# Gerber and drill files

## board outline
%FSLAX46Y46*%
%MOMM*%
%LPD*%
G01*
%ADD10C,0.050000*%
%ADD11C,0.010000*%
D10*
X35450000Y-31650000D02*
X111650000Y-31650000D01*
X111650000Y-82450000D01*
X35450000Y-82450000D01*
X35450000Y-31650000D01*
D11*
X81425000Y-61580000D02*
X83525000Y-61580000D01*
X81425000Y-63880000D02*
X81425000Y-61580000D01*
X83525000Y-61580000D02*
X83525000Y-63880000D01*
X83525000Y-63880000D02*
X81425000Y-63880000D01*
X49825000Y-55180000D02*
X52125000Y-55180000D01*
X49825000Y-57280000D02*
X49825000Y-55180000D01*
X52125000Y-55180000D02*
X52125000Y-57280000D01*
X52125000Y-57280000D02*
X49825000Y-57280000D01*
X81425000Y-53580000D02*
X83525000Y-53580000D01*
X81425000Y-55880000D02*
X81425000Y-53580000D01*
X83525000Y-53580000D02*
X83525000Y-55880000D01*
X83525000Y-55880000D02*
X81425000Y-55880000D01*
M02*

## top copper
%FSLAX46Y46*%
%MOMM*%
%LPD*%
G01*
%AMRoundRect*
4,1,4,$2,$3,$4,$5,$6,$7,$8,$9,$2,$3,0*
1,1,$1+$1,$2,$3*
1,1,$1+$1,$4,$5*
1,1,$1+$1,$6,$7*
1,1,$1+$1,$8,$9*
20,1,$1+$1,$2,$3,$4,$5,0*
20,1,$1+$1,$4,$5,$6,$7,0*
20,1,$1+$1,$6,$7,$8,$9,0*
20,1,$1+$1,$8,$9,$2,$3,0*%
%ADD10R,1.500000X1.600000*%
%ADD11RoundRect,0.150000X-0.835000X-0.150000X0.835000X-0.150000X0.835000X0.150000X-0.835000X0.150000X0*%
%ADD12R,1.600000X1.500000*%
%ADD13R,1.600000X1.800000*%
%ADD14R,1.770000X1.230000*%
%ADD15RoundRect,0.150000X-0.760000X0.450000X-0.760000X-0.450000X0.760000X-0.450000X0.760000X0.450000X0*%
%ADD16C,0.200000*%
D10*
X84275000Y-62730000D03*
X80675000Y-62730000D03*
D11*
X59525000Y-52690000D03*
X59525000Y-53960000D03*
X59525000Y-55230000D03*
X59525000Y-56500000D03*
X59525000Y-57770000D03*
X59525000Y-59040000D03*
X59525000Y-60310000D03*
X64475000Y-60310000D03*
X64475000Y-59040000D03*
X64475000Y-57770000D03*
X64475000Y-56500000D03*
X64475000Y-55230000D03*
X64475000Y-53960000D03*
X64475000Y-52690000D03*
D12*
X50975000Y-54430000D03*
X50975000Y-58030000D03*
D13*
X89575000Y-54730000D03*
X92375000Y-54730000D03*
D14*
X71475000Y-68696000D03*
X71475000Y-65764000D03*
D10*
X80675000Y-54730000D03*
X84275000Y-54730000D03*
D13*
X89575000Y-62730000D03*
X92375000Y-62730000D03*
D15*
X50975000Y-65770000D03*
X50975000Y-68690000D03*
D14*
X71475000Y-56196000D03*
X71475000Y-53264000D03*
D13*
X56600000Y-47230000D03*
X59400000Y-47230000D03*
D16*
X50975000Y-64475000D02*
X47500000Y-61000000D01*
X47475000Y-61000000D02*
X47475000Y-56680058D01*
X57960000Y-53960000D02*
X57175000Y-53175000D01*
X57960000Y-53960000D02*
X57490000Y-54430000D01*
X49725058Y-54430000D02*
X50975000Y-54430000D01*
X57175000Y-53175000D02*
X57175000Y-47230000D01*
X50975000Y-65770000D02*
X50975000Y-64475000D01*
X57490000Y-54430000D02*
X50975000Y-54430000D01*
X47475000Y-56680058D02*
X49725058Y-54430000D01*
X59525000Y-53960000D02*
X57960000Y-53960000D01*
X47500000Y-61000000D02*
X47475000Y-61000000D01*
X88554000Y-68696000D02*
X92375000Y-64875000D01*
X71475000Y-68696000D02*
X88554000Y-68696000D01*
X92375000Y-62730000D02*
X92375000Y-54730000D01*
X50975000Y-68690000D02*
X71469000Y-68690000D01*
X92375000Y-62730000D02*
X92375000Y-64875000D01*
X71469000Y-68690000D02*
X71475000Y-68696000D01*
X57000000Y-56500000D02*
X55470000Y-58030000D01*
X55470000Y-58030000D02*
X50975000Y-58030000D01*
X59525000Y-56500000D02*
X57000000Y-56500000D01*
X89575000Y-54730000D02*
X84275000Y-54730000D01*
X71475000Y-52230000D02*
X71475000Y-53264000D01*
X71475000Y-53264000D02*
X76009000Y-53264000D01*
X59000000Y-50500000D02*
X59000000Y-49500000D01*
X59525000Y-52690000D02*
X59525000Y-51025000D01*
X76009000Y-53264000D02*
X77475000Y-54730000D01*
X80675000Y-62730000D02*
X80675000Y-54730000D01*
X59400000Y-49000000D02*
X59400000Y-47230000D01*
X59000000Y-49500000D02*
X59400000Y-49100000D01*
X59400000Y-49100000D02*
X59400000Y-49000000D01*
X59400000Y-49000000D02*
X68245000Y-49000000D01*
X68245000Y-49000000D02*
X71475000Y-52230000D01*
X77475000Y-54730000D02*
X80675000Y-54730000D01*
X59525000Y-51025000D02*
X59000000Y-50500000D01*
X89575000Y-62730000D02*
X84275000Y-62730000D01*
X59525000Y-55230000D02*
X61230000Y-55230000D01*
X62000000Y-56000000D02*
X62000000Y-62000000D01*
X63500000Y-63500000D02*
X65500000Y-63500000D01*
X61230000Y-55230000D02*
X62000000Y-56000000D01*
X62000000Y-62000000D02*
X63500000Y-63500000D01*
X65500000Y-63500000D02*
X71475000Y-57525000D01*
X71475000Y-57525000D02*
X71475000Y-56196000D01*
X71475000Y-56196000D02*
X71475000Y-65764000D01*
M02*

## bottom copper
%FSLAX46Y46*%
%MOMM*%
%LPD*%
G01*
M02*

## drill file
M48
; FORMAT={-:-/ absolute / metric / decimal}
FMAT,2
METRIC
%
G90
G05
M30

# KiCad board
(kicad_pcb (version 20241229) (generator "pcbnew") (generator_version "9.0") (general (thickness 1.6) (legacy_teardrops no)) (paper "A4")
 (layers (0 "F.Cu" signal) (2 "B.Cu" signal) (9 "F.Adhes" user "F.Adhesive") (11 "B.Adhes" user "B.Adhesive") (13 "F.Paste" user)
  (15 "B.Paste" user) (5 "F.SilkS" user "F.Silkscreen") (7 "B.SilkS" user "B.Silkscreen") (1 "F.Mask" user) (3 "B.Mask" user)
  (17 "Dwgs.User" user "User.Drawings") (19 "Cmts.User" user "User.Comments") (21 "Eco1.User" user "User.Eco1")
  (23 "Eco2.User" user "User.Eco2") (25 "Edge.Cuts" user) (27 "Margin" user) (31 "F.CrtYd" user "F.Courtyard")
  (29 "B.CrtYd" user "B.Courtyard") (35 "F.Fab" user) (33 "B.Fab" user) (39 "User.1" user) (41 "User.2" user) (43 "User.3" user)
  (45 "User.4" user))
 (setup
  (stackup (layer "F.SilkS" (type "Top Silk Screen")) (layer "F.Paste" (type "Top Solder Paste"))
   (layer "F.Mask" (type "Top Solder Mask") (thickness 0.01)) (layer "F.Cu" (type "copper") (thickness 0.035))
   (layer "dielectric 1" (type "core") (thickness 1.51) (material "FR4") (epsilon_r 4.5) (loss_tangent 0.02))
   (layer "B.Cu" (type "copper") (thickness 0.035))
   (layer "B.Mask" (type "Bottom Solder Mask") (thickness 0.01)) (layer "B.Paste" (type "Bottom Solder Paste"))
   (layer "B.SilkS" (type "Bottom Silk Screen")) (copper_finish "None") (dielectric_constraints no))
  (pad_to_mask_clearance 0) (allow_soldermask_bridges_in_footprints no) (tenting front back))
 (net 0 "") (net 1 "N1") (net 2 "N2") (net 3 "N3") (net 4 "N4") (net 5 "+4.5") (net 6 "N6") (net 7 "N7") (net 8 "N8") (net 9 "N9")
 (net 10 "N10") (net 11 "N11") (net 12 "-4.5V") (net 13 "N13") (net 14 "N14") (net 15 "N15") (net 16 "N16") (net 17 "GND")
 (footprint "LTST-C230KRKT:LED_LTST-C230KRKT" (layer "F.Cu") (at 82.475 62.73)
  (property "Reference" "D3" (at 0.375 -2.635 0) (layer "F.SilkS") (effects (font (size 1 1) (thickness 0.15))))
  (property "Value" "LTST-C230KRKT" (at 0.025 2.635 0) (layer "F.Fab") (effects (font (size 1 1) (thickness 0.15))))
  (fp_line (start -1.05 -1.15) (end 1.05 -1.15) (stroke (width 0.01) (type solid)) (layer "Edge.Cuts"))
  (fp_line (start -1.05 1.15) (end -1.05 -1.15) (stroke (width 0.01) (type solid)) (layer "Edge.Cuts"))
  (fp_line (start 1.05 -1.15) (end 1.05 1.15) (stroke (width 0.01) (type solid)) (layer "Edge.Cuts"))
  (fp_line (start 1.05 1.15) (end -1.05 1.15) (stroke (width 0.01) (type solid)) (layer "Edge.Cuts"))
  (pad "A" smd rect (at 1.8 0) (size 1.5 1.6) (layers "F.Cu" "F.Mask" "F.Paste") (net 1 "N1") (solder_mask_margin 0.102))
  (pad "C" smd rect (at -1.8 0) (size 1.5 1.6) (layers "F.Cu" "F.Mask" "F.Paste") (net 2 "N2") (solder_mask_margin 0.102)))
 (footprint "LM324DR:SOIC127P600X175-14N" (layer "F.Cu") (at 62 56.5)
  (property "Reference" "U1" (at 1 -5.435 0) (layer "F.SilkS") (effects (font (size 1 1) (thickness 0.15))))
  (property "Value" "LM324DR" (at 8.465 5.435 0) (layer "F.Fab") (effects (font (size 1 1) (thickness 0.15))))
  (pad "1" smd roundrect (at -2.475 -3.81) (size 1.97 0.6) (layers "F.Cu" "F.Mask" "F.Paste") (roundrect_rratio 0.25) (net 2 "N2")
   (solder_mask_margin 0.102))
  (pad "2" smd roundrect (at -2.475 -2.54) (size 1.97 0.6) (layers "F.Cu" "F.Mask" "F.Paste") (roundrect_rratio 0.25) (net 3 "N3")
   (solder_mask_margin 0.102))
  (pad "3" smd roundrect (at -2.475 -1.27) (size 1.97 0.6) (layers "F.Cu" "F.Mask" "F.Paste") (roundrect_rratio 0.25) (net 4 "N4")
   (solder_mask_margin 0.102))
  (pad "4" smd roundrect (at -2.475 0) (size 1.97 0.6) (layers "F.Cu" "F.Mask" "F.Paste") (roundrect_rratio 0.25) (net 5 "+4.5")
   (solder_mask_margin 0.102))
  (pad "5" smd roundrect (at -2.475 1.27) (size 1.97 0.6) (layers "F.Cu" "F.Mask" "F.Paste") (roundrect_rratio 0.25) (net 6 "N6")
   (solder_mask_margin 0.102))
  (pad "6" smd roundrect (at -2.475 2.54) (size 1.97 0.6) (layers "F.Cu" "F.Mask" "F.Paste") (roundrect_rratio 0.25) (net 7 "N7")
   (solder_mask_margin 0.102))
  (pad "7" smd roundrect (at -2.475 3.81) (size 1.97 0.6) (layers "F.Cu" "F.Mask" "F.Paste") (roundrect_rratio 0.25) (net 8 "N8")
   (solder_mask_margin 0.102))
  (pad "8" smd roundrect (at 2.475 3.81) (size 1.97 0.6) (layers "F.Cu" "F.Mask" "F.Paste") (roundrect_rratio 0.25) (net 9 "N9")
   (solder_mask_margin 0.102))
  (pad "9" smd roundrect (at 2.475 2.54) (size 1.97 0.6) (layers "F.Cu" "F.Mask" "F.Paste") (roundrect_rratio 0.25) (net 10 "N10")
   (solder_mask_margin 0.102))
  (pad "10" smd roundrect (at 2.475 1.27) (size 1.97 0.6) (layers "F.Cu" "F.Mask" "F.Paste") (roundrect_rratio 0.25) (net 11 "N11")
   (solder_mask_margin 0.102))
  (pad "11" smd roundrect (at 2.475 0) (size 1.97 0.6) (layers "F.Cu" "F.Mask" "F.Paste") (roundrect_rratio 0.25) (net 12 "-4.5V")
   (solder_mask_margin 0.102))
  (pad "12" smd roundrect (at 2.475 -1.27) (size 1.97 0.6) (layers "F.Cu" "F.Mask" "F.Paste") (roundrect_rratio 0.25) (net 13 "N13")
   (solder_mask_margin 0.102))
  (pad "13" smd roundrect (at 2.475 -2.54) (size 1.97 0.6) (layers "F.Cu" "F.Mask" "F.Paste") (roundrect_rratio 0.25) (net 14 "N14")
   (solder_mask_margin 0.102))
  (pad "14" smd roundrect (at 2.475 -3.81) (size 1.97 0.6) (layers "F.Cu" "F.Mask" "F.Paste") (roundrect_rratio 0.25) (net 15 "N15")
   (solder_mask_margin 0.102)))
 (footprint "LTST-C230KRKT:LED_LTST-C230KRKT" (layer "F.Cu") (at 50.975 56.23 90)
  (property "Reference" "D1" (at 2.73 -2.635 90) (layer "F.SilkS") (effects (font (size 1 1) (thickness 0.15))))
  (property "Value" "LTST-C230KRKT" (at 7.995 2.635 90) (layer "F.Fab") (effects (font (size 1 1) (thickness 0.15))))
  (fp_line (start 1.05 -1.15) (end 1.05 1.15) (stroke (width 0.01) (type solid)) (layer "Edge.Cuts"))
  (fp_line (start -1.05 -1.15) (end 1.05 -1.15) (stroke (width 0.01) (type solid)) (layer "Edge.Cuts"))
  (fp_line (start 1.05 1.15) (end -1.05 1.15) (stroke (width 0.01) (type solid)) (layer "Edge.Cuts"))
  (fp_line (start -1.05 1.15) (end -1.05 -1.15) (stroke (width 0.01) (type solid)) (layer "Edge.Cuts"))
  (pad "A" smd rect (at 1.8 0 90) (size 1.5 1.6) (layers "F.Cu" "F.Mask" "F.Paste") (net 3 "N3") (solder_mask_margin 0.102))
  (pad "C" smd rect (at -1.8 0 90) (size 1.5 1.6) (layers "F.Cu" "F.Mask" "F.Paste") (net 5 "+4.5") (solder_mask_margin 0.102)))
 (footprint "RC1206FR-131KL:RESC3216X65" (layer "F.Cu") (at 90.975 54.73)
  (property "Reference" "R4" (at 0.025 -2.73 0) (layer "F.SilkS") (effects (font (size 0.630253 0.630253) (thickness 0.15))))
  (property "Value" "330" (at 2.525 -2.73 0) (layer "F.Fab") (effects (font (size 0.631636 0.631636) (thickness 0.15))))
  (pad "1" smd rect (at -1.4 0) (size 1.6 1.8) (layers "F.Cu" "F.Mask" "F.Paste") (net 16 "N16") (solder_mask_margin 0.102))
  (pad "2" smd rect (at 1.4 0) (size 1.6 1.8) (layers "F.Cu" "F.Mask" "F.Paste") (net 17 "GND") (solder_mask_margin 0.102)))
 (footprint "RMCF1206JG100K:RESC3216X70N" (layer "F.Cu") (at 71.475 67.23 90)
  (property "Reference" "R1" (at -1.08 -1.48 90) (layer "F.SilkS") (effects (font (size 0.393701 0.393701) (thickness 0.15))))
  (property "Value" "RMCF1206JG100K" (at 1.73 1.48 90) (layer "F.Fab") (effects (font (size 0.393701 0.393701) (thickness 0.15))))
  (pad "1" smd rect (at -1.466 0 90) (size 1.23 1.77) (layers "F.Cu" "F.Mask" "F.Paste") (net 17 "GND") (solder_mask_margin 0.102))
  (pad "2" smd rect (at 1.466 0 90) (size 1.23 1.77) (layers "F.Cu" "F.Mask" "F.Paste") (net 4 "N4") (solder_mask_margin 0.102)))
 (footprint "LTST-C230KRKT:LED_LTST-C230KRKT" (layer "F.Cu") (at 82.475 54.73 180)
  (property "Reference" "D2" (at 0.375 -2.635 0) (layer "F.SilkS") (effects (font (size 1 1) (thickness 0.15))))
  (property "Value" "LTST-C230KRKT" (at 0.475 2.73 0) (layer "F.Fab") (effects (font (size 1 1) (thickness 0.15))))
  (fp_line (start 1.05 1.15) (end -1.05 1.15) (stroke (width 0.01) (type solid)) (layer "Edge.Cuts"))
  (fp_line (start 1.05 -1.15) (end 1.05 1.15) (stroke (width 0.01) (type solid)) (layer "Edge.Cuts"))
  (fp_line (start -1.05 1.15) (end -1.05 -1.15) (stroke (width 0.01) (type solid)) (layer "Edge.Cuts"))
  (fp_line (start -1.05 -1.15) (end 1.05 -1.15) (stroke (width 0.01) (type solid)) (layer "Edge.Cuts"))
  (pad "A" smd rect (at 1.8 0 180) (size 1.5 1.6) (layers "F.Cu" "F.Mask" "F.Paste") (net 2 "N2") (solder_mask_margin 0.102))
  (pad "C" smd rect (at -1.8 0 180) (size 1.5 1.6) (layers "F.Cu" "F.Mask" "F.Paste") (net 16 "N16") (solder_mask_margin 0.102)))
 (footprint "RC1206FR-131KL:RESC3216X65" (layer "F.Cu") (at 90.975 62.73)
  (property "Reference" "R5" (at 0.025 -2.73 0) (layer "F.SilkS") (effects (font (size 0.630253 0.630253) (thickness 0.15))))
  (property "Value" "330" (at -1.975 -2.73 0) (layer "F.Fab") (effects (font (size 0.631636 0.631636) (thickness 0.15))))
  (pad "1" smd rect (at -1.4 0) (size 1.6 1.8) (layers "F.Cu" "F.Mask" "F.Paste") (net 1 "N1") (solder_mask_margin 0.102))
  (pad "2" smd rect (at 1.4 0) (size 1.6 1.8) (layers "F.Cu" "F.Mask" "F.Paste") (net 17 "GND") (solder_mask_margin 0.102)))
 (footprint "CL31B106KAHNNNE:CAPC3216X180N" (layer "F.Cu") (at 50.975 67.23 -90)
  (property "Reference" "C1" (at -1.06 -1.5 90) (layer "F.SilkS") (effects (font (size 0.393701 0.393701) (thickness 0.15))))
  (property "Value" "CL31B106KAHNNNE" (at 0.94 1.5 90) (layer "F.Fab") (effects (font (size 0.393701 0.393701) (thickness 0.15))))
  (pad "1" smd roundrect (at -1.46 0 270) (size 1.2 1.82) (layers "F.Cu" "F.Mask" "F.Paste") (roundrect_rratio 0.125) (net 3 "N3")
   (solder_mask_margin 0.102))
  (pad "2" smd roundrect (at 1.46 0 270) (size 1.2 1.82) (layers "F.Cu" "F.Mask" "F.Paste") (roundrect_rratio 0.125) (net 17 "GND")
   (solder_mask_margin 0.102)))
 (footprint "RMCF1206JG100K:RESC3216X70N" (layer "F.Cu") (at 71.475 54.73 90)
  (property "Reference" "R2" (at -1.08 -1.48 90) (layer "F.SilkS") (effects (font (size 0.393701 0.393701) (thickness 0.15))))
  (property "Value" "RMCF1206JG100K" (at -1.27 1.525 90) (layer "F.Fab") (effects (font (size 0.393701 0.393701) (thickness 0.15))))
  (pad "1" smd rect (at -1.466 0 90) (size 1.23 1.77) (layers "F.Cu" "F.Mask" "F.Paste") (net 4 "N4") (solder_mask_margin 0.102))
  (pad "2" smd rect (at 1.466 0 90) (size 1.23 1.77) (layers "F.Cu" "F.Mask" "F.Paste") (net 2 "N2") (solder_mask_margin 0.102)))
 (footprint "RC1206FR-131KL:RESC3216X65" (layer "F.Cu") (at 58 47.23)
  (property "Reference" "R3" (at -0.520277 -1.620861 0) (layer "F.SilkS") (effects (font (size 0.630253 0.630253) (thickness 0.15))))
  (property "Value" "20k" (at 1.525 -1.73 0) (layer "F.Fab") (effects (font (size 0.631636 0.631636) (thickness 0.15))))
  (pad "1" smd rect (at -1.4 0) (size 1.6 1.8) (layers "F.Cu" "F.Mask" "F.Paste") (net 3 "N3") (solder_mask_margin 0.102))
  (pad "2" smd rect (at 1.4 0) (size 1.6 1.8) (layers "F.Cu" "F.Mask" "F.Paste") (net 2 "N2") (solder_mask_margin 0.102)))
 (gr_rect (start 35.45 31.65) (end 111.65 82.45) (stroke (width 0.05) (type solid)) (fill no) (layer "Edge.Cuts"))
 (segment (start 50.975 64.475) (end 47.5 61) (width 0.2) (layer "F.Cu") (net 3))
 (segment (start 47.475 61) (end 47.475 56.680058) (width 0.2) (layer "F.Cu") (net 3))
 (segment (start 57.96 53.96) (end 57.175 53.175) (width 0.2) (layer "F.Cu") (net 3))
 (segment (start 57.96 53.96) (end 57.49 54.43) (width 0.2) (layer "F.Cu") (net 3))
 (segment (start 49.725058 54.43) (end 50.975 54.43) (width 0.2) (layer "F.Cu") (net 3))
 (segment (start 57.175 53.175) (end 57.175 47.23) (width 0.2) (layer "F.Cu") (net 3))
 (segment (start 50.975 65.77) (end 50.975 64.475) (width 0.2) (layer "F.Cu") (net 3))
 (segment (start 57.49 54.43) (end 50.975 54.43) (width 0.2) (layer "F.Cu") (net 3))
 (segment (start 47.475 56.680058) (end 49.725058 54.43) (width 0.2) (layer "F.Cu") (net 3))
 (segment (start 59.525 53.96) (end 57.96 53.96) (width 0.2) (layer "F.Cu") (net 3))
 (segment (start 47.5 61) (end 47.475 61) (width 0.2) (layer "F.Cu") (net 3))
 (segment (start 88.554 68.696) (end 92.375 64.875) (width 0.2) (layer "F.Cu") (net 17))
 (segment (start 71.475 68.696) (end 88.554 68.696) (width 0.2) (layer "F.Cu") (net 17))
 (segment (start 92.375 62.73) (end 92.375 54.73) (width 0.2) (layer "F.Cu") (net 17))
 (segment (start 50.975 68.69) (end 71.469 68.69) (width 0.2) (layer "F.Cu") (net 17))
 (segment (start 92.375 62.73) (end 92.375 64.875) (width 0.2) (layer "F.Cu") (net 17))
 (segment (start 71.469 68.69) (end 71.475 68.696) (width 0.2) (layer "F.Cu") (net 17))
 (segment (start 57 56.5) (end 55.47 58.03) (width 0.2) (layer "F.Cu") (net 5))
 (segment (start 55.47 58.03) (end 50.975 58.03) (width 0.2) (layer "F.Cu") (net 5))
 (segment (start 59.525 56.5) (end 57 56.5) (width 0.2) (layer "F.Cu") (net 5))
 (segment (start 89.575 54.73) (end 84.275 54.73) (width 0.2) (layer "F.Cu") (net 16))
 (segment (start 71.475 52.23) (end 71.475 53.264) (width 0.2) (layer "F.Cu") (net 2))
 (segment (start 71.475 53.264) (end 76.009 53.264) (width 0.2) (layer "F.Cu") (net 2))
 (segment (start 59 50.5) (end 59 49.5) (width 0.2) (layer "F.Cu") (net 2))
 (segment (start 59.525 52.69) (end 59.525 51.025) (width 0.2) (layer "F.Cu") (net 2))
 (segment (start 76.009 53.264) (end 77.475 54.73) (width 0.2) (layer "F.Cu") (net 2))
 (segment (start 80.675 62.73) (end 80.675 54.73) (width 0.2) (layer "F.Cu") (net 2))
 (segment (start 59.4 49) (end 59.4 47.23) (width 0.2) (layer "F.Cu") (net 2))
 (segment (start 59 49.5) (end 59.4 49.1) (width 0.2) (layer "F.Cu") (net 2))
 (segment (start 59.4 49.1) (end 59.4 49) (width 0.2) (layer "F.Cu") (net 2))
 (segment (start 59.4 49) (end 68.245 49) (width 0.2) (layer "F.Cu") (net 2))
 (segment (start 68.245 49) (end 71.475 52.23) (width 0.2) (layer "F.Cu") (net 2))
 (segment (start 77.475 54.73) (end 80.675 54.73) (width 0.2) (layer "F.Cu") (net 2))
 (segment (start 59.525 51.025) (end 59 50.5) (width 0.2) (layer "F.Cu") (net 2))
 (segment (start 89.575 62.73) (end 84.275 62.73) (width 0.2) (layer "F.Cu") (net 1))
 (segment (start 59.525 55.23) (end 61.23 55.23) (width 0.2) (layer "F.Cu") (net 4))
 (segment (start 62 56) (end 62 62) (width 0.2) (layer "F.Cu") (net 4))
 (segment (start 63.5 63.5) (end 65.5 63.5) (width 0.2) (layer "F.Cu") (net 4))
 (segment (start 61.23 55.23) (end 62 56) (width 0.2) (layer "F.Cu") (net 4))
 (segment (start 62 62) (end 63.5 63.5) (width 0.2) (layer "F.Cu") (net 4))
 (segment (start 65.5 63.5) (end 71.475 57.525) (width 0.2) (layer "F.Cu") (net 4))
 (segment (start 71.475 57.525) (end 71.475 56.196) (width 0.2) (layer "F.Cu") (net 4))
 (segment (start 71.475 56.196) (end 71.475 65.764) (width 0.2) (layer "F.Cu") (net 4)))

